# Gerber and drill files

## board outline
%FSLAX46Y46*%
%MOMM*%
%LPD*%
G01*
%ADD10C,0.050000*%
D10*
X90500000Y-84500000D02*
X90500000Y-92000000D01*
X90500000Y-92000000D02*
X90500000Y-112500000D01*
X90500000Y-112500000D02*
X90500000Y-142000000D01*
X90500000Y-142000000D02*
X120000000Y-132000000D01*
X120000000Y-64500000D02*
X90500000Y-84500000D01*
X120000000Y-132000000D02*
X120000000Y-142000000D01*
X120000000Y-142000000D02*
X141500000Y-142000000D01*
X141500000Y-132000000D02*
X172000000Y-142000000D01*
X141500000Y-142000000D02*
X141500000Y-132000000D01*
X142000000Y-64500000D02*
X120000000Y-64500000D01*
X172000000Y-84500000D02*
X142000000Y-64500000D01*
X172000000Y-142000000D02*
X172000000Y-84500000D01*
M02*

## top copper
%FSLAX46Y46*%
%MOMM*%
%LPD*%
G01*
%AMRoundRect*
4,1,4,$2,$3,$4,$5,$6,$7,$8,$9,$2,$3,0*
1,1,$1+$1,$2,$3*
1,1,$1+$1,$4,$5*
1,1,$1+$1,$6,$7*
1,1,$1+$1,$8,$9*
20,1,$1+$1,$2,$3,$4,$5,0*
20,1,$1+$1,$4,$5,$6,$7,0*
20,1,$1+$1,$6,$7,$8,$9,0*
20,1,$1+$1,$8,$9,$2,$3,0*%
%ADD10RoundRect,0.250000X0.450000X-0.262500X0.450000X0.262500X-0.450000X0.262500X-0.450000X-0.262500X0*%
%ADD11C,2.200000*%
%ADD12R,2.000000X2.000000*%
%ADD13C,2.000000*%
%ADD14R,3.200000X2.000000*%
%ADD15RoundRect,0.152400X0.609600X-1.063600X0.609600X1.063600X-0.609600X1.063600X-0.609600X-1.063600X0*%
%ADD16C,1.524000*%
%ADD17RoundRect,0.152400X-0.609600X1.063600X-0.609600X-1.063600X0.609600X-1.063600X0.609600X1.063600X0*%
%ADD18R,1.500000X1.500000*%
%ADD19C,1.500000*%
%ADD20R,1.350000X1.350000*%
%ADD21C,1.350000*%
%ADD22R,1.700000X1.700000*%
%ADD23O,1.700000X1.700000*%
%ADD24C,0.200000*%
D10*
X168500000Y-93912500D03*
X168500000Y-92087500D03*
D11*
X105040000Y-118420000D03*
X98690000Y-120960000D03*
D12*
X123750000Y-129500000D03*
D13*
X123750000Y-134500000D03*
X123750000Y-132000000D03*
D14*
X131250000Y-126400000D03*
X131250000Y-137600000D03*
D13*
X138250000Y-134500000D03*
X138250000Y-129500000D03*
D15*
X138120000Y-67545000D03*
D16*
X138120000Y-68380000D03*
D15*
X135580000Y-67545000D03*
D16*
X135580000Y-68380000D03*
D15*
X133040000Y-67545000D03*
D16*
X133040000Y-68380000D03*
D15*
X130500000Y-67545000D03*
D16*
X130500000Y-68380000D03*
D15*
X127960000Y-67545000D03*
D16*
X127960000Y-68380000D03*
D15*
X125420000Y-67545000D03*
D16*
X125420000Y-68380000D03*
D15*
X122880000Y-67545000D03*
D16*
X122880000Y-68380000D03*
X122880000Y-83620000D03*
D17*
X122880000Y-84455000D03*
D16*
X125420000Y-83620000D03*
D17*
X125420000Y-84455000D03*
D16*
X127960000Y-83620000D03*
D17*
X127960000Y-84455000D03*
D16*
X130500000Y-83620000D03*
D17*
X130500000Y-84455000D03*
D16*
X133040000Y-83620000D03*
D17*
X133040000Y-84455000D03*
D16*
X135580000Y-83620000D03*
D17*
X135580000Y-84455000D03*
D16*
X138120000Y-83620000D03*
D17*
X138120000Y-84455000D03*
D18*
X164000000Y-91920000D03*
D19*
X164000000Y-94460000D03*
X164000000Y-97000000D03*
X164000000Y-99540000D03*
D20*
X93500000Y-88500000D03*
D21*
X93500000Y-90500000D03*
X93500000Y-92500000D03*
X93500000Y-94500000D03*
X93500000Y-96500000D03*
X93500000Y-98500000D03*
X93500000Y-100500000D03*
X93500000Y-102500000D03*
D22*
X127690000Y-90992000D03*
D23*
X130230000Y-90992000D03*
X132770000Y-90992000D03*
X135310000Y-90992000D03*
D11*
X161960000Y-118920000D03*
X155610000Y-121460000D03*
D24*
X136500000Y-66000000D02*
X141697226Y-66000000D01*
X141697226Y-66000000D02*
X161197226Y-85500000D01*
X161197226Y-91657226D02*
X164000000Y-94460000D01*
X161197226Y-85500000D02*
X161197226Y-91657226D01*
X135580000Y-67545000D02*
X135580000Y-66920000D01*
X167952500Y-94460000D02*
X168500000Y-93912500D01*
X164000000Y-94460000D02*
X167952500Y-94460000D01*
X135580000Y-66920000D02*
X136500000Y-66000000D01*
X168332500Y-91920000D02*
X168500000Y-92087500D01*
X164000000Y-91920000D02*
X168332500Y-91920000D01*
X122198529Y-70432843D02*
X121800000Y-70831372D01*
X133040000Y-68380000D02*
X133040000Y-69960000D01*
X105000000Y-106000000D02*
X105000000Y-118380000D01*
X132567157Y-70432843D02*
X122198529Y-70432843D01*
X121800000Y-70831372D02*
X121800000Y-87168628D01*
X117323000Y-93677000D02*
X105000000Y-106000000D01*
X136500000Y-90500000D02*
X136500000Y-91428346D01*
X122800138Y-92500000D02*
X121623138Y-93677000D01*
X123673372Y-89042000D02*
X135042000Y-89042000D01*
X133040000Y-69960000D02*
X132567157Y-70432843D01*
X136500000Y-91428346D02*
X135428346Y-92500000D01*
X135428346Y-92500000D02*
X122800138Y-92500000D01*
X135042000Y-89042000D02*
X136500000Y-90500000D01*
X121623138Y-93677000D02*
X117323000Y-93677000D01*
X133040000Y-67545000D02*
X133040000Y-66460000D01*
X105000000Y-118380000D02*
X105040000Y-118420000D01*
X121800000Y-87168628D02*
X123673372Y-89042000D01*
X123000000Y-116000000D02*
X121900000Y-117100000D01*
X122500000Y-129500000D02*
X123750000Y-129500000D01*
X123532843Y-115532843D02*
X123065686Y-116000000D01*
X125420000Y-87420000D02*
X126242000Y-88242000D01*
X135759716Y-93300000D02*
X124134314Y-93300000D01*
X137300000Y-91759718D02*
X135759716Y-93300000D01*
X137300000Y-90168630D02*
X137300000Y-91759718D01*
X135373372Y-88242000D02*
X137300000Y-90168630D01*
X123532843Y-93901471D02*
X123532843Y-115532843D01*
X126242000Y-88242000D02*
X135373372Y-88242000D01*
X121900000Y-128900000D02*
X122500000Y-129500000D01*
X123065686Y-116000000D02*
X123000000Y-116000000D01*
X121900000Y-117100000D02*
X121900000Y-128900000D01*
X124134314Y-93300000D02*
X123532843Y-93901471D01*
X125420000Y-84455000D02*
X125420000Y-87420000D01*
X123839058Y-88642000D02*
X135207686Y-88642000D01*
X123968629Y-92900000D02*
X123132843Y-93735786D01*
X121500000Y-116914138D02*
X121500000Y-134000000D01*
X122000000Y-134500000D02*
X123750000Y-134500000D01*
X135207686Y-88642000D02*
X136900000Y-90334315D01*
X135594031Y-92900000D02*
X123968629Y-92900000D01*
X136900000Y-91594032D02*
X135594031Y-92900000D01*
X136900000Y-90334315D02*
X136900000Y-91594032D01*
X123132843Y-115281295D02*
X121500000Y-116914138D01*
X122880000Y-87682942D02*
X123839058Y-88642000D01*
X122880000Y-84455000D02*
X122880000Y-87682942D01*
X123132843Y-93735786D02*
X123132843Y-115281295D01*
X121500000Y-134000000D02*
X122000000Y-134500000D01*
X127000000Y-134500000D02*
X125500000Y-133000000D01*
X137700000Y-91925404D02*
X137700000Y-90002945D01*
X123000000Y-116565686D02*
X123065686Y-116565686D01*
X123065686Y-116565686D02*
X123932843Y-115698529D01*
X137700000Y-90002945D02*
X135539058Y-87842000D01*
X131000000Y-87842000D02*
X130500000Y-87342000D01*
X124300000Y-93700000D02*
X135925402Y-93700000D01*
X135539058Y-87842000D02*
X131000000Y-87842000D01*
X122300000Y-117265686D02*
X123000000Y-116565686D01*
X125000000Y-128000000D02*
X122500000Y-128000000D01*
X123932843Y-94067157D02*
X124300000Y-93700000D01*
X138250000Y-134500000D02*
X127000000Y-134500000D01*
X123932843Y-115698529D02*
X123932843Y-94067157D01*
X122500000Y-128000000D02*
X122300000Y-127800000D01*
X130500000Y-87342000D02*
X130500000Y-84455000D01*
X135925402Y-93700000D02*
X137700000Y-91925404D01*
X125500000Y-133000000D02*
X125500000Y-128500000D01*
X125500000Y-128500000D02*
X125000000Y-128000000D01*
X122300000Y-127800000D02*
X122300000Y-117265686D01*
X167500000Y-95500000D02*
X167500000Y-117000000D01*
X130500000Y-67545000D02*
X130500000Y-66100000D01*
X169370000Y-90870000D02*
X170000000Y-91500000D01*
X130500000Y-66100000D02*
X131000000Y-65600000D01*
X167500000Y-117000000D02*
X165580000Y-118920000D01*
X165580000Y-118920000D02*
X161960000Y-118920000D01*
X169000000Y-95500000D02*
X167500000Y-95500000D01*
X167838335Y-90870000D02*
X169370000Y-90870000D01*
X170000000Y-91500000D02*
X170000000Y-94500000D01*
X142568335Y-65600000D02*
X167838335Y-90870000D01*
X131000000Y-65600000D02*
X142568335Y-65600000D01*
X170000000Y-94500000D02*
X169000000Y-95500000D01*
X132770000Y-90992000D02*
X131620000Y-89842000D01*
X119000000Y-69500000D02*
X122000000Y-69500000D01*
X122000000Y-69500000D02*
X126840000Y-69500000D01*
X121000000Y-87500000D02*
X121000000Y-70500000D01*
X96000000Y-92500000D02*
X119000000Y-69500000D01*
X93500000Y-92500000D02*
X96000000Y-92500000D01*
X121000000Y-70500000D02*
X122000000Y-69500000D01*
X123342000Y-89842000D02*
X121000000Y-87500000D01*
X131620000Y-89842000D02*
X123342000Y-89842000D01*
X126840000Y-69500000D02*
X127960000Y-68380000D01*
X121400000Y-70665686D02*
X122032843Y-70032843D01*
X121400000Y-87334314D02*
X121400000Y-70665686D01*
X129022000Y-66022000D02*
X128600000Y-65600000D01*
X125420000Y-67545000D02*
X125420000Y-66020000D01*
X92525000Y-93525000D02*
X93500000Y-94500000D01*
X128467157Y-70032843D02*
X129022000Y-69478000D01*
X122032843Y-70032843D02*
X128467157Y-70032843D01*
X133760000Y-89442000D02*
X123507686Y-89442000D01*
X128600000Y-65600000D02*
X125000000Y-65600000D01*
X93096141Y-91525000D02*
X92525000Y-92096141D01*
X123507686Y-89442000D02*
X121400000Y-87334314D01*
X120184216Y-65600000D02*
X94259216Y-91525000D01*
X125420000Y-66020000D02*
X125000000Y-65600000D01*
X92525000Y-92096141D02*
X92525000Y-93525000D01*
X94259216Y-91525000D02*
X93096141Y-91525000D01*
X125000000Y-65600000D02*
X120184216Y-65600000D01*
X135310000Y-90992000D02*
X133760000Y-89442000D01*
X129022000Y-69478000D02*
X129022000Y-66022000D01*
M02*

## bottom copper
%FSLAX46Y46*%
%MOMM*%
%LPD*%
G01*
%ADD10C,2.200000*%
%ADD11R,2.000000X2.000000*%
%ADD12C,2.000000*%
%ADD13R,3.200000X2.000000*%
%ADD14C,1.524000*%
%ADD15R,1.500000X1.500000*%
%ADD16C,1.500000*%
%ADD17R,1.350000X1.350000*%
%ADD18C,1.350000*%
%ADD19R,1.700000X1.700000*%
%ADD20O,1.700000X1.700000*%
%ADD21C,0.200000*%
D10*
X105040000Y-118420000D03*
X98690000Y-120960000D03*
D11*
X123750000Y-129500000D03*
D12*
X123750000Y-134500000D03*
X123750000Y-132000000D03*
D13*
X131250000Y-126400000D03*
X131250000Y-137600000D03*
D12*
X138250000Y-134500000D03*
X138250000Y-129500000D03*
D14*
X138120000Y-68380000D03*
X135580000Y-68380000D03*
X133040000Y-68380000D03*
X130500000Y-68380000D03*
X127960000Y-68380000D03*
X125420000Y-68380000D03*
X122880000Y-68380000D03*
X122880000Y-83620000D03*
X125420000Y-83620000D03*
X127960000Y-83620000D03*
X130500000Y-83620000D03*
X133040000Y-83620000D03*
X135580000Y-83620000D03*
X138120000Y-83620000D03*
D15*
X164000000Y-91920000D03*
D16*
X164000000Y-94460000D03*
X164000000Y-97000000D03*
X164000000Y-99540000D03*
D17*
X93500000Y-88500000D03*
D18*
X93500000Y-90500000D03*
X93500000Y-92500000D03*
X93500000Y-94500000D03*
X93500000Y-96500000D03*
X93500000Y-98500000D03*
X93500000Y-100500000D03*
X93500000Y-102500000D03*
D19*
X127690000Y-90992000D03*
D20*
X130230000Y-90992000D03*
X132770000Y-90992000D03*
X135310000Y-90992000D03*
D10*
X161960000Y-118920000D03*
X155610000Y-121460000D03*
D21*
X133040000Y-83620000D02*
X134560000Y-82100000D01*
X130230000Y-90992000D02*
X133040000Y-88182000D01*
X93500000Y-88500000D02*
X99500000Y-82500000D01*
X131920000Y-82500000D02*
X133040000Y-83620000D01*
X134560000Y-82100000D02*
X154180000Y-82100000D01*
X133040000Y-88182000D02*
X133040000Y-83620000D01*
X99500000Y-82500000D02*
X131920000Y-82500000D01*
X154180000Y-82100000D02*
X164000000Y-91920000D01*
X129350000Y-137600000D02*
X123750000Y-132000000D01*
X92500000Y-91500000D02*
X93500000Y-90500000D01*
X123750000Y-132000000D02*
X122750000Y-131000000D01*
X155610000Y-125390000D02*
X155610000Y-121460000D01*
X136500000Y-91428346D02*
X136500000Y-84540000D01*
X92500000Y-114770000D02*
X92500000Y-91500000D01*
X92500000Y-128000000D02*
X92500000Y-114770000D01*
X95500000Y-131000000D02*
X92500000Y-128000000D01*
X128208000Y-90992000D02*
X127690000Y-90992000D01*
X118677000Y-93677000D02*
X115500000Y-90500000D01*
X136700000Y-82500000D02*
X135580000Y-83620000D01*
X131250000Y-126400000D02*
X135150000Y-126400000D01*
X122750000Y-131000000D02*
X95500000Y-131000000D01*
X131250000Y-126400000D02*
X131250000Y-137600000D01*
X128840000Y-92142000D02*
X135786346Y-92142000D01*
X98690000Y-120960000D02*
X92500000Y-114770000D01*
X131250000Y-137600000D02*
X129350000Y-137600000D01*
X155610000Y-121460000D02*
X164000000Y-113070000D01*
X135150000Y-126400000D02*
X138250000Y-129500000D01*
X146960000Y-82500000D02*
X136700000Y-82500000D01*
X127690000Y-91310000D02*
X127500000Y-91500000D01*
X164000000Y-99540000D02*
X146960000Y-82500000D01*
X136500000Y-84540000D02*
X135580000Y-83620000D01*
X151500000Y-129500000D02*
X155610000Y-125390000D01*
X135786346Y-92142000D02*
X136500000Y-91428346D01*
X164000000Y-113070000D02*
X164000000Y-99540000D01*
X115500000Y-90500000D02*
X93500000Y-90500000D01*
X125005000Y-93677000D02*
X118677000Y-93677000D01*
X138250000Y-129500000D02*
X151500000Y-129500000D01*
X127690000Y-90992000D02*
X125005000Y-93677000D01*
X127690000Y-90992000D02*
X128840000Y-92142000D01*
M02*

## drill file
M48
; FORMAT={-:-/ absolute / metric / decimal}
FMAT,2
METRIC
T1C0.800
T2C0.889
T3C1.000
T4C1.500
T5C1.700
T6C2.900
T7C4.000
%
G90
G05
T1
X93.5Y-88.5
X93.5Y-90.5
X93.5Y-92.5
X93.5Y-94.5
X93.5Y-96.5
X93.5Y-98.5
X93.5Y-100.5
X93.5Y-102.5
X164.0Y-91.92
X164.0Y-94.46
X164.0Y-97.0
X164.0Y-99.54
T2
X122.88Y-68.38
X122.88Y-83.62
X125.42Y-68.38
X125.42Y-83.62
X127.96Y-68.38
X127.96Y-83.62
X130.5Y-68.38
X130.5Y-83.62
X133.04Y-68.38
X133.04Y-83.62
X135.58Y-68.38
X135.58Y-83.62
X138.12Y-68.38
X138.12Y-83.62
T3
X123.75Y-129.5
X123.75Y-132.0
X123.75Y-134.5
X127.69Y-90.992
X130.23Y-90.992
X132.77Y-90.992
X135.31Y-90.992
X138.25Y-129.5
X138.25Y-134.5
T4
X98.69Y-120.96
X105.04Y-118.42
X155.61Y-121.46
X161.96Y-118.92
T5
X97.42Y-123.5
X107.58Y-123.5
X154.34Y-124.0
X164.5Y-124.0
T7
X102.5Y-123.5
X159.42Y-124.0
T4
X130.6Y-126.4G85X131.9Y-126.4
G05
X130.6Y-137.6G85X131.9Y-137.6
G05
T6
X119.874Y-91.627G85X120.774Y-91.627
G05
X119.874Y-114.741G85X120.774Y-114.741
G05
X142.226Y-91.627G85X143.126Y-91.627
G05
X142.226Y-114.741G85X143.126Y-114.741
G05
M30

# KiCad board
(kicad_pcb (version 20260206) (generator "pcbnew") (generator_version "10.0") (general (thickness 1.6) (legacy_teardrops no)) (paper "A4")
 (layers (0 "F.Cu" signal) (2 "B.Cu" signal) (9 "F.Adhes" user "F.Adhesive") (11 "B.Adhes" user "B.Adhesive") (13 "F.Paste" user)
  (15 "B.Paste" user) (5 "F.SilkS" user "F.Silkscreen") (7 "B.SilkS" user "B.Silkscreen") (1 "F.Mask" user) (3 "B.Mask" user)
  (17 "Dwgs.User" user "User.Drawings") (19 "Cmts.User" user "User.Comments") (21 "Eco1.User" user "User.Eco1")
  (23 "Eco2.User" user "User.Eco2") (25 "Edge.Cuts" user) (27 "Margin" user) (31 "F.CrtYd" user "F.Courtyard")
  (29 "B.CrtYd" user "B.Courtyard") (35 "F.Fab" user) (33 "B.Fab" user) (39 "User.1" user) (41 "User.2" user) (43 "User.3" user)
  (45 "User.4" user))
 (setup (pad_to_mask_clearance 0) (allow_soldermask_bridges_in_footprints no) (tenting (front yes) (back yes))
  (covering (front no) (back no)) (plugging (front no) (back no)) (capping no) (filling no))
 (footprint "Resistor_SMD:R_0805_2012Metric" (layer "F.Cu") (at 168.5 93 90)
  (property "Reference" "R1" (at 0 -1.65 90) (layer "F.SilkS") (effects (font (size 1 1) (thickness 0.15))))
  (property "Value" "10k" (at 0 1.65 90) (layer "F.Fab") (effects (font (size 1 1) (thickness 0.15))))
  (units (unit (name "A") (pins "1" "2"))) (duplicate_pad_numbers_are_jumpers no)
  (pad "1" smd roundrect (at -0.9125 0 90) (size 1.025 1.4) (layers "F.Cu" "F.Mask" "F.Paste") (roundrect_rratio 0.243902)
   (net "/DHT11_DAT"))
  (pad "2" smd roundrect (at 0.9125 0 90) (size 1.025 1.4) (layers "F.Cu" "F.Mask" "F.Paste") (roundrect_rratio 0.243902) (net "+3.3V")))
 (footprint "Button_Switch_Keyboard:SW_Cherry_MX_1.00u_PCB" (layer "F.Cu") (at 105.04 118.42)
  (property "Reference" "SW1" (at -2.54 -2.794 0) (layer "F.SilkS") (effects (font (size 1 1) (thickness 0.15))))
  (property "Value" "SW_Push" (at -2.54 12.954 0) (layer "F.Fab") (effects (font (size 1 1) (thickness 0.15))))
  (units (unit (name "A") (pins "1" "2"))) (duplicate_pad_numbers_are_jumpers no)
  (pad "" np_thru_hole circle (at -7.62 5.08) (size 1.7 1.7) (drill 1.7) (layers "*.Cu" "*.Mask"))
  (pad "" np_thru_hole circle (at -2.54 5.08) (size 4 4) (drill 4) (layers "*.Cu" "*.Mask"))
  (pad "" np_thru_hole circle (at 2.54 5.08) (size 1.7 1.7) (drill 1.7) (layers "*.Cu" "*.Mask"))
  (pad "1" thru_hole circle (at 0 0) (size 2.2 2.2) (drill 1.5) (layers "*.Cu" "*.Mask") (remove_unused_layers no) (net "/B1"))
  (pad "2" thru_hole circle (at -6.35 2.54) (size 2.2 2.2) (drill 1.5) (layers "*.Cu" "*.Mask") (remove_unused_layers no) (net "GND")))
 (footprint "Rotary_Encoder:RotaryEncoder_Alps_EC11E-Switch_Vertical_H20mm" (layer "F.Cu") (at 123.75 129.5)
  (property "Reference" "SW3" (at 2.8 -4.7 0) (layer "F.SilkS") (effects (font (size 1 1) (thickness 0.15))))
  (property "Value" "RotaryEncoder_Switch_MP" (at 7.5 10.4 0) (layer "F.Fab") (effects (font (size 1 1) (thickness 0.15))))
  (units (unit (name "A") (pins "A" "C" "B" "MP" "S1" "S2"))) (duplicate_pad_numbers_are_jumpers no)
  (pad "A" thru_hole rect (at 0 0) (size 2 2) (drill 1) (layers "*.Cu" "*.Mask") (remove_unused_layers no) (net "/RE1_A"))
  (pad "B" thru_hole circle (at 0 5) (size 2 2) (drill 1) (layers "*.Cu" "*.Mask") (remove_unused_layers no) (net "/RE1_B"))
  (pad "C" thru_hole circle (at 0 2.5) (size 2 2) (drill 1) (layers "*.Cu" "*.Mask") (remove_unused_layers no) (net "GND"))
  (pad "MP" thru_hole rect (at 7.5 -3.1) (size 3.2 2) (drill oval 2.8 1.5) (layers "*.Cu" "*.Mask") (remove_unused_layers no) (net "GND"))
  (pad "MP" thru_hole rect (at 7.5 8.1) (size 3.2 2) (drill oval 2.8 1.5) (layers "*.Cu" "*.Mask") (remove_unused_layers no) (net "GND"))
  (pad "S1" thru_hole circle (at 14.5 5) (size 2 2) (drill 1) (layers "*.Cu" "*.Mask") (remove_unused_layers no) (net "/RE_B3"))
  (pad "S2" thru_hole circle (at 14.5 0) (size 2 2) (drill 1) (layers "*.Cu" "*.Mask") (remove_unused_layers no) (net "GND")))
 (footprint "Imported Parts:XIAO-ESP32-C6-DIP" (layer "F.Cu") (at 130.5 76)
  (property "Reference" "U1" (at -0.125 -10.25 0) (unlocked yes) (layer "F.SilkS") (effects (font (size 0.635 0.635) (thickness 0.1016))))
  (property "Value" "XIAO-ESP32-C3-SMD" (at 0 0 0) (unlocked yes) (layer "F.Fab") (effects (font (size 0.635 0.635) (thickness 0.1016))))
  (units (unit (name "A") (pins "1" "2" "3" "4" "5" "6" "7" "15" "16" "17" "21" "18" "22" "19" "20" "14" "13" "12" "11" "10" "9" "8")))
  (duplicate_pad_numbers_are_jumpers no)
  (pad "1" smd roundrect (at 7.62 -8.455 90) (size 2.432 1.524) (layers "F.Cu" "F.Mask") (roundrect_rratio 0.1)
   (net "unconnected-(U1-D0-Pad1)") (thermal_bridge_angle 45))
  (pad "1" thru_hole circle (at 7.62 -7.62 90) (size 1.524 1.524) (drill 0.889) (layers "*.Cu" "*.Mask") (remove_unused_layers no)
   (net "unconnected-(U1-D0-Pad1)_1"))
  (pad "2" smd roundrect (at 5.08 -8.455 90) (size 2.432 1.524) (layers "F.Cu" "F.Mask") (roundrect_rratio 0.1) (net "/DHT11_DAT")
   (thermal_bridge_angle 45))
  (pad "2" thru_hole circle (at 5.08 -7.62 90) (size 1.524 1.524) (drill 0.889) (layers "*.Cu" "*.Mask") (remove_unused_layers no)
   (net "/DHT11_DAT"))
  (pad "3" smd roundrect (at 2.54 -8.455 90) (size 2.432 1.524) (layers "F.Cu" "F.Mask") (roundrect_rratio 0.1) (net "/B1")
   (thermal_bridge_angle 45))
  (pad "3" thru_hole circle (at 2.54 -7.62 90) (size 1.524 1.524) (drill 0.889) (layers "*.Cu" "*.Mask") (remove_unused_layers no)
   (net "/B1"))
  (pad "4" smd roundrect (at 0 -8.455 90) (size 2.432 1.524) (layers "F.Cu" "F.Mask") (roundrect_rratio 0.1) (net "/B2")
   (thermal_bridge_angle 45))
  (pad "4" thru_hole circle (at 0 -7.62 90) (size 1.524 1.524) (drill 0.889) (layers "*.Cu" "*.Mask") (remove_unused_layers no) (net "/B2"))
  (pad "5" smd roundrect (at -2.54 -8.455 90) (size 2.432 1.524) (layers "F.Cu" "F.Mask") (roundrect_rratio 0.1) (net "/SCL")
   (thermal_bridge_angle 45))
  (pad "5" thru_hole circle (at -2.54 -7.62 90) (size 1.524 1.524) (drill 0.889) (layers "*.Cu" "*.Mask") (remove_unused_layers no)
   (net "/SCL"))
  (pad "6" smd roundrect (at -5.08 -8.455 90) (size 2.432 1.524) (layers "F.Cu" "F.Mask") (roundrect_rratio 0.1) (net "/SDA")
   (thermal_bridge_angle 45))
  (pad "6" thru_hole circle (at -5.08 -7.62 90) (size 1.524 1.524) (drill 0.889) (layers "*.Cu" "*.Mask") (remove_unused_layers no)
   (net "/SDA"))
  (pad "7" smd roundrect (at -7.62 -8.455 90) (size 2.432 1.524) (layers "F.Cu" "F.Mask") (roundrect_rratio 0.1)
   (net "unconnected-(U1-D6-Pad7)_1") (thermal_bridge_angle 45))
  (pad "7" thru_hole circle (at -7.62 -7.62 90) (size 1.524 1.524) (drill 0.889) (layers "*.Cu" "*.Mask") (remove_unused_layers no)
   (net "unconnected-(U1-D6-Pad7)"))
  (pad "8" thru_hole circle (at -7.62 7.62 270) (size 1.524 1.524) (drill 0.889) (layers "*.Cu" "*.Mask") (remove_unused_layers no)
   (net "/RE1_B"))
  (pad "8" smd roundrect (at -7.62 8.455 270) (size 2.432 1.524) (layers "F.Cu" "F.Mask") (roundrect_rratio 0.1) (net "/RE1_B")
   (thermal_bridge_angle 45))
  (pad "9" thru_hole circle (at -5.08 7.62 270) (size 1.524 1.524) (drill 0.889) (layers "*.Cu" "*.Mask") (remove_unused_layers no)
   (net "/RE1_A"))
  (pad "9" smd roundrect (at -5.08 8.455 270) (size 2.432 1.524) (layers "F.Cu" "F.Mask") (roundrect_rratio 0.1) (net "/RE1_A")
   (thermal_bridge_angle 45))
  (pad "10" thru_hole circle (at -2.54 7.62 270) (size 1.524 1.524) (drill 0.889) (layers "*.Cu" "*.Mask") (remove_unused_layers no)
   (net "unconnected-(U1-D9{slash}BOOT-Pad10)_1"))
  (pad "10" smd roundrect (at -2.54 8.455 270) (size 2.432 1.524) (layers "F.Cu" "F.Mask") (roundrect_rratio 0.1)
   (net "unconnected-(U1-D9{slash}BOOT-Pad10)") (thermal_bridge_angle 45))
  (pad "11" thru_hole circle (at 0 7.62 270) (size 1.524 1.524) (drill 0.889) (layers "*.Cu" "*.Mask") (remove_unused_layers no)
   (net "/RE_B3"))
  (pad "11" smd roundrect (at 0 8.455 270) (size 2.432 1.524) (layers "F.Cu" "F.Mask") (roundrect_rratio 0.1) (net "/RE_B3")
   (thermal_bridge_angle 45))
  (pad "12" thru_hole circle (at 2.54 7.62 270) (size 1.524 1.524) (drill 0.889) (layers "*.Cu" "*.Mask") (remove_unused_layers no)
   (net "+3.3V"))
  (pad "12" smd roundrect (at 2.54 8.455 270) (size 2.432 1.524) (layers "F.Cu" "F.Mask") (roundrect_rratio 0.1) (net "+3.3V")
   (thermal_bridge_angle 45))
  (pad "13" thru_hole circle (at 5.08 7.62 270) (size 1.524 1.524) (drill 0.889) (layers "*.Cu" "*.Mask") (remove_unused_layers no)
   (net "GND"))
  (pad "13" smd roundrect (at 5.08 8.455 270) (size 2.432 1.524) (layers "F.Cu" "F.Mask") (roundrect_rratio 0.1) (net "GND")
   (thermal_bridge_angle 45))
  (pad "14" thru_hole circle (at 7.62 7.62 270) (size 1.524 1.524) (drill 0.889) (layers "*.Cu" "*.Mask") (remove_unused_layers no)
   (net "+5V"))
  (pad "14" smd roundrect (at 7.62 8.455 270) (size 2.432 1.524) (layers "F.Cu" "F.Mask") (roundrect_rratio 0.1) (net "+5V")
   (thermal_bridge_angle 45)))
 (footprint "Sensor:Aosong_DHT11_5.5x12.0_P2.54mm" (layer "F.Cu") (at 164 91.92)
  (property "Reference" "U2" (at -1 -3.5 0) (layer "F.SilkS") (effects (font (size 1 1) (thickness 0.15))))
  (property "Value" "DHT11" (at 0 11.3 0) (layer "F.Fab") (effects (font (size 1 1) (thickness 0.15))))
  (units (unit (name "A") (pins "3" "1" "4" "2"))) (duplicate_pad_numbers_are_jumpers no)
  (pad "1" thru_hole rect (at 0 0) (size 1.5 1.5) (drill 0.8) (layers "*.Cu" "*.Mask") (remove_unused_layers no) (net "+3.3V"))
  (pad "2" thru_hole circle (at 0 2.54) (size 1.5 1.5) (drill 0.8) (layers "*.Cu" "*.Mask") (remove_unused_layers no) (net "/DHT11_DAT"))
  (pad "3" thru_hole circle (at 0 5.08) (size 1.5 1.5) (drill 0.8) (layers "*.Cu" "*.Mask") (remove_unused_layers no)
   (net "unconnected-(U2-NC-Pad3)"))
  (pad "4" thru_hole circle (at 0 7.62) (size 1.5 1.5) (drill 0.8) (layers "*.Cu" "*.Mask") (remove_unused_layers no) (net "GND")))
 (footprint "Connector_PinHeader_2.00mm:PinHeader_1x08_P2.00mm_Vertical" (layer "F.Cu") (at 93.5 88.5)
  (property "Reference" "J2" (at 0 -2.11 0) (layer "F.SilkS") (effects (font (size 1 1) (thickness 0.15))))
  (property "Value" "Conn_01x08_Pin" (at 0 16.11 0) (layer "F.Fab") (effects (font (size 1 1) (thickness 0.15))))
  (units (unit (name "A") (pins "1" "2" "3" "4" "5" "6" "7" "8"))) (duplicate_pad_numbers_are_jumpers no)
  (pad "1" thru_hole rect (at 0 0) (size 1.35 1.35) (drill 0.8) (layers "*.Cu" "*.Mask") (remove_unused_layers no) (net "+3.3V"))
  (pad "2" thru_hole circle (at 0 2) (size 1.35 1.35) (drill 0.8) (layers "*.Cu" "*.Mask") (remove_unused_layers no) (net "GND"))
  (pad "3" thru_hole circle (at 0 4) (size 1.35 1.35) (drill 0.8) (layers "*.Cu" "*.Mask") (remove_unused_layers no) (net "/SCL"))
  (pad "4" thru_hole circle (at 0 6) (size 1.35 1.35) (drill 0.8) (layers "*.Cu" "*.Mask") (remove_unused_layers no) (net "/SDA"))
  (pad "5" thru_hole circle (at 0 8) (size 1.35 1.35) (drill 0.8) (layers "*.Cu" "*.Mask") (remove_unused_layers no)
   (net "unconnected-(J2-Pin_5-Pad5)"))
  (pad "6" thru_hole circle (at 0 10) (size 1.35 1.35) (drill 0.8) (layers "*.Cu" "*.Mask") (remove_unused_layers no)
   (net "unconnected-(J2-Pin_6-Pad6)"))
  (pad "7" thru_hole circle (at 0 12) (size 1.35 1.35) (drill 0.8) (layers "*.Cu" "*.Mask") (remove_unused_layers no)
   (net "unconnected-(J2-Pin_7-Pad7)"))
  (pad "8" thru_hole circle (at 0 14) (size 1.35 1.35) (drill 0.8) (layers "*.Cu" "*.Mask") (remove_unused_layers no)
   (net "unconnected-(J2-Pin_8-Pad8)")))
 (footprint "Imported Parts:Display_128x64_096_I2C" (layer "F.Cu") (at 131.5 90.992)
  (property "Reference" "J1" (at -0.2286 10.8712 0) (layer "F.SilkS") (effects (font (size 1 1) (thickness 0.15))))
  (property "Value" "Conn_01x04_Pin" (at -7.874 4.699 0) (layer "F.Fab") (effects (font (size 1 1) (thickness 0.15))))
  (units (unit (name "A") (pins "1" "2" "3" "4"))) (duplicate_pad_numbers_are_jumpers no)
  (pad "" np_thru_hole oval (at -11.176 0.635) (size 3.8 2.9) (drill oval 3.8 2.9) (layers "*.Cu" "*.Mask"))
  (pad "" np_thru_hole oval (at -11.176 23.749) (size 3.8 2.9) (drill oval 3.8 2.9) (layers "*.Cu" "*.Mask"))
  (pad "" np_thru_hole oval (at 11.176 0.635) (size 3.8 2.9) (drill oval 3.8 2.9) (layers "*.Cu" "*.Mask"))
  (pad "" np_thru_hole oval (at 11.176 23.749) (size 3.8 2.9) (drill oval 3.8 2.9) (layers "*.Cu" "*.Mask"))
  (pad "1" thru_hole rect (at -3.81 0 90) (size 1.7 1.7) (drill 1) (layers "*.Cu" "*.Mask") (remove_unused_layers no) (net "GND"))
  (pad "2" thru_hole oval (at -1.27 0 90) (size 1.7 1.7) (drill 1) (layers "*.Cu" "*.Mask") (remove_unused_layers no) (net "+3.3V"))
  (pad "3" thru_hole oval (at 1.27 0 90) (size 1.7 1.7) (drill 1) (layers "*.Cu" "*.Mask") (remove_unused_layers no) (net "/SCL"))
  (pad "4" thru_hole oval (at 3.81 0 90) (size 1.7 1.7) (drill 1) (layers "*.Cu" "*.Mask") (remove_unused_layers no) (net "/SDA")))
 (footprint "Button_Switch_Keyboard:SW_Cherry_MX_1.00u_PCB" (layer "F.Cu") (at 161.96 118.92)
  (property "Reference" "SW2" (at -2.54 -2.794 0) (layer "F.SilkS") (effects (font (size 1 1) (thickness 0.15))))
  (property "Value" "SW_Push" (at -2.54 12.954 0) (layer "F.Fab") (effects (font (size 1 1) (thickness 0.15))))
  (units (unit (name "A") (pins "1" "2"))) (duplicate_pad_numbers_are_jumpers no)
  (pad "" np_thru_hole circle (at -7.62 5.08) (size 1.7 1.7) (drill 1.7) (layers "*.Cu" "*.Mask"))
  (pad "" np_thru_hole circle (at -2.54 5.08) (size 4 4) (drill 4) (layers "*.Cu" "*.Mask"))
  (pad "" np_thru_hole circle (at 2.54 5.08) (size 1.7 1.7) (drill 1.7) (layers "*.Cu" "*.Mask"))
  (pad "1" thru_hole circle (at 0 0) (size 2.2 2.2) (drill 1.5) (layers "*.Cu" "*.Mask") (remove_unused_layers no) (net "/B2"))
  (pad "2" thru_hole circle (at -6.35 2.54) (size 2.2 2.2) (drill 1.5) (layers "*.Cu" "*.Mask") (remove_unused_layers no) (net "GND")))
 (gr_line (start 90.5 84.5) (end 90.5 92) (stroke (width 0.05) (type default)) (layer "Edge.Cuts"))
 (gr_line (start 90.5 92) (end 90.5 112.5) (stroke (width 0.05) (type default)) (layer "Edge.Cuts"))
 (gr_line (start 90.5 112.5) (end 90.5 142) (stroke (width 0.05) (type default)) (layer "Edge.Cuts"))
 (gr_line (start 90.5 142) (end 120 132) (stroke (width 0.05) (type default)) (layer "Edge.Cuts"))
 (gr_line (start 120 64.5) (end 90.5 84.5) (stroke (width 0.05) (type default)) (layer "Edge.Cuts"))
 (gr_line (start 120 132) (end 120 142) (stroke (width 0.05) (type default)) (layer "Edge.Cuts"))
 (gr_line (start 120 142) (end 141.5 142) (stroke (width 0.05) (type default)) (layer "Edge.Cuts"))
 (gr_line (start 141.5 132) (end 172 142) (stroke (width 0.05) (type default)) (layer "Edge.Cuts"))
 (gr_line (start 141.5 142) (end 141.5 132) (stroke (width 0.05) (type default)) (layer "Edge.Cuts"))
 (gr_line (start 142 64.5) (end 120 64.5) (stroke (width 0.05) (type default)) (layer "Edge.Cuts"))
 (gr_line (start 172 84.5) (end 142 64.5) (stroke (width 0.05) (type default)) (layer "Edge.Cuts"))
 (gr_line (start 172 142) (end 172 84.5) (stroke (width 0.05) (type default)) (layer "Edge.Cuts"))
 (segment (start 136.5 66) (end 141.697226 66) (width 0.2) (layer "F.Cu") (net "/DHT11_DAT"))
 (segment (start 141.697226 66) (end 161.197226 85.5) (width 0.2) (layer "F.Cu") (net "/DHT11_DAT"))
 (segment (start 161.197226 91.657226) (end 164 94.46) (width 0.2) (layer "F.Cu") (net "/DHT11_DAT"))
 (segment (start 161.197226 85.5) (end 161.197226 91.657226) (width 0.2) (layer "F.Cu") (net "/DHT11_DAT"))
 (segment (start 135.58 67.545) (end 135.58 66.92) (width 0.2) (layer "F.Cu") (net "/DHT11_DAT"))
 (segment (start 167.9525 94.46) (end 168.5 93.9125) (width 0.2) (layer "F.Cu") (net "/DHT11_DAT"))
 (segment (start 164 94.46) (end 167.9525 94.46) (width 0.2) (layer "F.Cu") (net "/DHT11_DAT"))
 (segment (start 135.58 66.92) (end 136.5 66) (width 0.2) (layer "F.Cu") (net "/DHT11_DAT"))
 (segment (start 168.3325 91.92) (end 168.5 92.0875) (width 0.2) (layer "F.Cu") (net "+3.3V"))
 (segment (start 164 91.92) (end 168.3325 91.92) (width 0.2) (layer "F.Cu") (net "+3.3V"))
 (segment (start 133.04 83.62) (end 134.56 82.1) (width 0.2) (layer "B.Cu") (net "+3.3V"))
 (segment (start 130.23 90.992) (end 133.04 88.182) (width 0.2) (layer "B.Cu") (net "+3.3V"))
 (segment (start 93.5 88.5) (end 99.5 82.5) (width 0.2) (layer "B.Cu") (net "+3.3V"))
 (segment (start 131.92 82.5) (end 133.04 83.62) (width 0.2) (layer "B.Cu") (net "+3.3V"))
 (segment (start 134.56 82.1) (end 154.18 82.1) (width 0.2) (layer "B.Cu") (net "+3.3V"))
 (segment (start 133.04 88.182) (end 133.04 83.62) (width 0.2) (layer "B.Cu") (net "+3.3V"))
 (segment (start 99.5 82.5) (end 131.92 82.5) (width 0.2) (layer "B.Cu") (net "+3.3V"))
 (segment (start 154.18 82.1) (end 164 91.92) (width 0.2) (layer "B.Cu") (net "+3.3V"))
 (segment (start 122.198529 70.432843) (end 121.8 70.831372) (width 0.2) (layer "F.Cu") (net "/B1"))
 (segment (start 133.04 68.38) (end 133.04 69.96) (width 0.2) (layer "F.Cu") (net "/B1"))
 (segment (start 105 106) (end 105 118.38) (width 0.2) (layer "F.Cu") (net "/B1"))
 (segment (start 132.567157 70.432843) (end 122.198529 70.432843) (width 0.2) (layer "F.Cu") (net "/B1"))
 (segment (start 121.8 70.831372) (end 121.8 87.168628) (width 0.2) (layer "F.Cu") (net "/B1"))
 (segment (start 117.323 93.677) (end 105 106) (width 0.2) (layer "F.Cu") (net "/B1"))
 (segment (start 136.5 90.5) (end 136.5 91.428346) (width 0.2) (layer "F.Cu") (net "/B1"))
 (segment (start 122.800138 92.5) (end 121.623138 93.677) (width 0.2) (layer "F.Cu") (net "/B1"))
 (segment (start 123.673372 89.042) (end 135.042 89.042) (width 0.2) (layer "F.Cu") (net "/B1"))
 (segment (start 133.04 69.96) (end 132.567157 70.432843) (width 0.2) (layer "F.Cu") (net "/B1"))
 (segment (start 136.5 91.428346) (end 135.428346 92.5) (width 0.2) (layer "F.Cu") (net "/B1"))
 (segment (start 135.428346 92.5) (end 122.800138 92.5) (width 0.2) (layer "F.Cu") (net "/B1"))
 (segment (start 135.042 89.042) (end 136.5 90.5) (width 0.2) (layer "F.Cu") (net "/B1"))
 (segment (start 121.623138 93.677) (end 117.323 93.677) (width 0.2) (layer "F.Cu") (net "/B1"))
 (segment (start 133.04 67.545) (end 133.04 66.46) (width 0.2) (layer "F.Cu") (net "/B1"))
 (segment (start 105 118.38) (end 105.04 118.42) (width 0.2) (layer "F.Cu") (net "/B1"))
 (segment (start 121.8 87.168628) (end 123.673372 89.042) (width 0.2) (layer "F.Cu") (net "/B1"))
 (segment (start 129.35 137.6) (end 123.75 132) (width 0.2) (layer "B.Cu") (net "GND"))
 (segment (start 92.5 91.5) (end 93.5 90.5) (width 0.2) (layer "B.Cu") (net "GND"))
 (segment (start 123.75 132) (end 122.75 131) (width 0.2) (layer "B.Cu") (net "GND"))
 (segment (start 155.61 125.39) (end 155.61 121.46) (width 0.2) (layer "B.Cu") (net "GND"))
 (segment (start 136.5 91.428346) (end 136.5 84.54) (width 0.2) (layer "B.Cu") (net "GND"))
 (segment (start 92.5 114.77) (end 92.5 91.5) (width 0.2) (layer "B.Cu") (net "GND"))
 (segment (start 92.5 128) (end 92.5 114.77) (width 0.2) (layer "B.Cu") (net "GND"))
 (segment (start 95.5 131) (end 92.5 128) (width 0.2) (layer "B.Cu") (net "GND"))
 (segment (start 128.208 90.992) (end 127.69 90.992) (width 0.2) (layer "B.Cu") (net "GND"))
 (segment (start 118.677 93.677) (end 115.5 90.5) (width 0.2) (layer "B.Cu") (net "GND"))
 (segment (start 136.7 82.5) (end 135.58 83.62) (width 0.2) (layer "B.Cu") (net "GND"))
 (segment (start 131.25 126.4) (end 135.15 126.4) (width 0.2) (layer "B.Cu") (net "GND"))
 (segment (start 122.75 131) (end 95.5 131) (width 0.2) (layer "B.Cu") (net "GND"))
 (segment (start 131.25 126.4) (end 131.25 137.6) (width 0.2) (layer "B.Cu") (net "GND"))
 (segment (start 128.84 92.142) (end 135.786346 92.142) (width 0.2) (layer "B.Cu") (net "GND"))
 (segment (start 98.69 120.96) (end 92.5 114.77) (width 0.2) (layer "B.Cu") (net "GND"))
 (segment (start 131.25 137.6) (end 129.35 137.6) (width 0.2) (layer "B.Cu") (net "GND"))
 (segment (start 155.61 121.46) (end 164 113.07) (width 0.2) (layer "B.Cu") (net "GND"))
 (segment (start 135.15 126.4) (end 138.25 129.5) (width 0.2) (layer "B.Cu") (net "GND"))
 (segment (start 146.96 82.5) (end 136.7 82.5) (width 0.2) (layer "B.Cu") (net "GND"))
 (segment (start 127.69 91.31) (end 127.5 91.5) (width 0.2) (layer "B.Cu") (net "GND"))
 (segment (start 164 99.54) (end 146.96 82.5) (width 0.2) (layer "B.Cu") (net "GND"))
 (segment (start 136.5 84.54) (end 135.58 83.62) (width 0.2) (layer "B.Cu") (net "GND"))
 (segment (start 151.5 129.5) (end 155.61 125.39) (width 0.2) (layer "B.Cu") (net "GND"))
 (segment (start 135.786346 92.142) (end 136.5 91.428346) (width 0.2) (layer "B.Cu") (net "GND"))
 (segment (start 164 113.07) (end 164 99.54) (width 0.2) (layer "B.Cu") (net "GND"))
 (segment (start 115.5 90.5) (end 93.5 90.5) (width 0.2) (layer "B.Cu") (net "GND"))
 (segment (start 125.005 93.677) (end 118.677 93.677) (width 0.2) (layer "B.Cu") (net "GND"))
 (segment (start 138.25 129.5) (end 151.5 129.5) (width 0.2) (layer "B.Cu") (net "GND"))
 (segment (start 127.69 90.992) (end 125.005 93.677) (width 0.2) (layer "B.Cu") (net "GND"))
 (segment (start 127.69 90.992) (end 128.84 92.142) (width 0.2) (layer "B.Cu") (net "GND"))
 (segment (start 123 116) (end 121.9 117.1) (width 0.2) (layer "F.Cu") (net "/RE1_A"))
 (segment (start 122.5 129.5) (end 123.75 129.5) (width 0.2) (layer "F.Cu") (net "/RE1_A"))
 (segment (start 123.532843 115.532843) (end 123.065686 116) (width 0.2) (layer "F.Cu") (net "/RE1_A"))
 (segment (start 125.42 87.42) (end 126.242 88.242) (width 0.2) (layer "F.Cu") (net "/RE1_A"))
 (segment (start 135.759716 93.3) (end 124.134314 93.3) (width 0.2) (layer "F.Cu") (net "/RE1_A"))
 (segment (start 137.3 91.759718) (end 135.759716 93.3) (width 0.2) (layer "F.Cu") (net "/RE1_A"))
 (segment (start 137.3 90.16863) (end 137.3 91.759718) (width 0.2) (layer "F.Cu") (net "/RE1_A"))
 (segment (start 135.373372 88.242) (end 137.3 90.16863) (width 0.2) (layer "F.Cu") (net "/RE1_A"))
 (segment (start 123.532843 93.901471) (end 123.532843 115.532843) (width 0.2) (layer "F.Cu") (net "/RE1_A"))
 (segment (start 126.242 88.242) (end 135.373372 88.242) (width 0.2) (layer "F.Cu") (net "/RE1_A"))
 (segment (start 121.9 128.9) (end 122.5 129.5) (width 0.2) (layer "F.Cu") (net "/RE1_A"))
 (segment (start 123.065686 116) (end 123 116) (width 0.2) (layer "F.Cu") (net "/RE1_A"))
 (segment (start 121.9 117.1) (end 121.9 128.9) (width 0.2) (layer "F.Cu") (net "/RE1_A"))
 (segment (start 124.134314 93.3) (end 123.532843 93.901471) (width 0.2) (layer "F.Cu") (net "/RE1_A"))
 (segment (start 125.42 84.455) (end 125.42 87.42) (width 0.2) (layer "F.Cu") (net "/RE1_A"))
 (segment (start 123.839058 88.642) (end 135.207686 88.642) (width 0.2) (layer "F.Cu") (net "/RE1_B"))
 (segment (start 123.968629 92.9) (end 123.132843 93.735786) (width 0.2) (layer "F.Cu") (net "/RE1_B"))
 (segment (start 121.5 116.914138) (end 121.5 134) (width 0.2) (layer "F.Cu") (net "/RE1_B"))
 (segment (start 122 134.5) (end 123.75 134.5) (width 0.2) (layer "F.Cu") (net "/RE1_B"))
 (segment (start 135.207686 88.642) (end 136.9 90.334315) (width 0.2) (layer "F.Cu") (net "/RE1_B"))
 (segment (start 135.594031 92.9) (end 123.968629 92.9) (width 0.2) (layer "F.Cu") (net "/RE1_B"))
 (segment (start 136.9 91.594032) (end 135.594031 92.9) (width 0.2) (layer "F.Cu") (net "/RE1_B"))
 (segment (start 136.9 90.334315) (end 136.9 91.594032) (width 0.2) (layer "F.Cu") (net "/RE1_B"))
 (segment (start 123.132843 115.281295) (end 121.5 116.914138) (width 0.2) (layer "F.Cu") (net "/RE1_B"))
 (segment (start 122.88 87.682942) (end 123.839058 88.642) (width 0.2) (layer "F.Cu") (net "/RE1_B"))
 (segment (start 122.88 84.455) (end 122.88 87.682942) (width 0.2) (layer "F.Cu") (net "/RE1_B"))
 (segment (start 123.132843 93.735786) (end 123.132843 115.281295) (width 0.2) (layer "F.Cu") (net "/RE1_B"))
 (segment (start 121.5 134) (end 122 134.5) (width 0.2) (layer "F.Cu") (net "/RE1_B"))
 (segment (start 127 134.5) (end 125.5 133) (width 0.2) (layer "F.Cu") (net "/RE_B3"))
 (segment (start 137.7 91.925404) (end 137.7 90.002945) (width 0.2) (layer "F.Cu") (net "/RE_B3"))
 (segment (start 123 116.565686) (end 123.065686 116.565686) (width 0.2) (layer "F.Cu") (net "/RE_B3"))
 (segment (start 123.065686 116.565686) (end 123.932843 115.698529) (width 0.2) (layer "F.Cu") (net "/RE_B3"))
 (segment (start 137.7 90.002945) (end 135.539058 87.842) (width 0.2) (layer "F.Cu") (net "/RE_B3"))
 (segment (start 131 87.842) (end 130.5 87.342) (width 0.2) (layer "F.Cu") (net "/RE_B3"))
 (segment (start 124.3 93.7) (end 135.925402 93.7) (width 0.2) (layer "F.Cu") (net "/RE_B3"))
 (segment (start 135.539058 87.842) (end 131 87.842) (width 0.2) (layer "F.Cu") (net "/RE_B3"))
 (segment (start 122.3 117.265686) (end 123 116.565686) (width 0.2) (layer "F.Cu") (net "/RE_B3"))
 (segment (start 125 128) (end 122.5 128) (width 0.2) (layer "F.Cu") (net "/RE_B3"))
 (segment (start 123.932843 94.067157) (end 124.3 93.7) (width 0.2) (layer "F.Cu") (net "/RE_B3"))
 (segment (start 138.25 134.5) (end 127 134.5) (width 0.2) (layer "F.Cu") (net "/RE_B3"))
 (segment (start 123.932843 115.698529) (end 123.932843 94.067157) (width 0.2) (layer "F.Cu") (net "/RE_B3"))
 (segment (start 122.5 128) (end 122.3 127.8) (width 0.2) (layer "F.Cu") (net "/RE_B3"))
 (segment (start 130.5 87.342) (end 130.5 84.455) (width 0.2) (layer "F.Cu") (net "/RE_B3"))
 (segment (start 135.925402 93.7) (end 137.7 91.925404) (width 0.2) (layer "F.Cu") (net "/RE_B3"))
 (segment (start 125.5 133) (end 125.5 128.5) (width 0.2) (layer "F.Cu") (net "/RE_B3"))
 (segment (start 125.5 128.5) (end 125 128) (width 0.2) (layer "F.Cu") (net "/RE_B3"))
 (segment (start 122.3 127.8) (end 122.3 117.265686) (width 0.2) (layer "F.Cu") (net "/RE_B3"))
 (segment (start 167.5 95.5) (end 167.5 117) (width 0.2) (layer "F.Cu") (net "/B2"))
 (segment (start 130.5 67.545) (end 130.5 66.1) (width 0.2) (layer "F.Cu") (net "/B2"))
 (segment (start 169.37 90.87) (end 170 91.5) (width 0.2) (layer "F.Cu") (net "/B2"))
 (segment (start 130.5 66.1) (end 131 65.6) (width 0.2) (layer "F.Cu") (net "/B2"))
 (segment (start 167.5 117) (end 165.58 118.92) (width 0.2) (layer "F.Cu") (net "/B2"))
 (segment (start 165.58 118.92) (end 161.96 118.92) (width 0.2) (layer "F.Cu") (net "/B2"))
 (segment (start 169 95.5) (end 167.5 95.5) (width 0.2) (layer "F.Cu") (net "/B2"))
 (segment (start 167.838335 90.87) (end 169.37 90.87) (width 0.2) (layer "F.Cu") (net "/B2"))
 (segment (start 170 91.5) (end 170 94.5) (width 0.2) (layer "F.Cu") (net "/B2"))
 (segment (start 142.568335 65.6) (end 167.838335 90.87) (width 0.2) (layer "F.Cu") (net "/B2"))
 (segment (start 131 65.6) (end 142.568335 65.6) (width 0.2) (layer "F.Cu") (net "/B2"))
 (segment (start 170 94.5) (end 169 95.5) (width 0.2) (layer "F.Cu") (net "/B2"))
 (segment (start 132.77 90.992) (end 131.62 89.842) (width 0.2) (layer "F.Cu") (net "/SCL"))
 (segment (start 119 69.5) (end 122 69.5) (width 0.2) (layer "F.Cu") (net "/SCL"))
 (segment (start 122 69.5) (end 126.84 69.5) (width 0.2) (layer "F.Cu") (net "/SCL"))
 (segment (start 121 87.5) (end 121 70.5) (width 0.2) (layer "F.Cu") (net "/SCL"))
 (segment (start 96 92.5) (end 119 69.5) (width 0.2) (layer "F.Cu") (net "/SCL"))
 (segment (start 93.5 92.5) (end 96 92.5) (width 0.2) (layer "F.Cu") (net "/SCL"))
 (segment (start 121 70.5) (end 122 69.5) (width 0.2) (layer "F.Cu") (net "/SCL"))
 (segment (start 123.342 89.842) (end 121 87.5) (width 0.2) (layer "F.Cu") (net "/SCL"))
 (segment (start 131.62 89.842) (end 123.342 89.842) (width 0.2) (layer "F.Cu") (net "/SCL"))
 (segment (start 126.84 69.5) (end 127.96 68.38) (width 0.2) (layer "F.Cu") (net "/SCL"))
 (segment (start 121.4 70.665686) (end 122.032843 70.032843) (width 0.2) (layer "F.Cu") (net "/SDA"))
 (segment (start 121.4 87.334314) (end 121.4 70.665686) (width 0.2) (layer "F.Cu") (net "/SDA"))
 (segment (start 129.022 66.022) (end 128.6 65.6) (width 0.2) (layer "F.Cu") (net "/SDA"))
 (segment (start 125.42 67.545) (end 125.42 66.02) (width 0.2) (layer "F.Cu") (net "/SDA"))
 (segment (start 92.525 93.525) (end 93.5 94.5) (width 0.2) (layer "F.Cu") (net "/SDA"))
 (segment (start 128.467157 70.032843) (end 129.022 69.478) (width 0.2) (layer "F.Cu") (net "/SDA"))
 (segment (start 122.032843 70.032843) (end 128.467157 70.032843) (width 0.2) (layer "F.Cu") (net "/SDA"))
 (segment (start 133.76 89.442) (end 123.507686 89.442) (width 0.2) (layer "F.Cu") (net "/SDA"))
 (segment (start 128.6 65.6) (end 125 65.6) (width 0.2) (layer "F.Cu") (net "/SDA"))
 (segment (start 93.096141 91.525) (end 92.525 92.096141) (width 0.2) (layer "F.Cu") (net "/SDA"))
 (segment (start 123.507686 89.442) (end 121.4 87.334314) (width 0.2) (layer "F.Cu") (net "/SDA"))
 (segment (start 120.184216 65.6) (end 94.259216 91.525) (width 0.2) (layer "F.Cu") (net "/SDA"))
 (segment (start 125.42 66.02) (end 125 65.6) (width 0.2) (layer "F.Cu") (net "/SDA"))
 (segment (start 92.525 92.096141) (end 92.525 93.525) (width 0.2) (layer "F.Cu") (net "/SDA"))
 (segment (start 94.259216 91.525) (end 93.096141 91.525) (width 0.2) (layer "F.Cu") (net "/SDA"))
 (segment (start 125 65.6) (end 120.184216 65.6) (width 0.2) (layer "F.Cu") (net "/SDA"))
 (segment (start 135.31 90.992) (end 133.76 89.442) (width 0.2) (layer "F.Cu") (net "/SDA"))
 (segment (start 129.022 69.478) (end 129.022 66.022) (width 0.2) (layer "F.Cu") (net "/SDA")))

